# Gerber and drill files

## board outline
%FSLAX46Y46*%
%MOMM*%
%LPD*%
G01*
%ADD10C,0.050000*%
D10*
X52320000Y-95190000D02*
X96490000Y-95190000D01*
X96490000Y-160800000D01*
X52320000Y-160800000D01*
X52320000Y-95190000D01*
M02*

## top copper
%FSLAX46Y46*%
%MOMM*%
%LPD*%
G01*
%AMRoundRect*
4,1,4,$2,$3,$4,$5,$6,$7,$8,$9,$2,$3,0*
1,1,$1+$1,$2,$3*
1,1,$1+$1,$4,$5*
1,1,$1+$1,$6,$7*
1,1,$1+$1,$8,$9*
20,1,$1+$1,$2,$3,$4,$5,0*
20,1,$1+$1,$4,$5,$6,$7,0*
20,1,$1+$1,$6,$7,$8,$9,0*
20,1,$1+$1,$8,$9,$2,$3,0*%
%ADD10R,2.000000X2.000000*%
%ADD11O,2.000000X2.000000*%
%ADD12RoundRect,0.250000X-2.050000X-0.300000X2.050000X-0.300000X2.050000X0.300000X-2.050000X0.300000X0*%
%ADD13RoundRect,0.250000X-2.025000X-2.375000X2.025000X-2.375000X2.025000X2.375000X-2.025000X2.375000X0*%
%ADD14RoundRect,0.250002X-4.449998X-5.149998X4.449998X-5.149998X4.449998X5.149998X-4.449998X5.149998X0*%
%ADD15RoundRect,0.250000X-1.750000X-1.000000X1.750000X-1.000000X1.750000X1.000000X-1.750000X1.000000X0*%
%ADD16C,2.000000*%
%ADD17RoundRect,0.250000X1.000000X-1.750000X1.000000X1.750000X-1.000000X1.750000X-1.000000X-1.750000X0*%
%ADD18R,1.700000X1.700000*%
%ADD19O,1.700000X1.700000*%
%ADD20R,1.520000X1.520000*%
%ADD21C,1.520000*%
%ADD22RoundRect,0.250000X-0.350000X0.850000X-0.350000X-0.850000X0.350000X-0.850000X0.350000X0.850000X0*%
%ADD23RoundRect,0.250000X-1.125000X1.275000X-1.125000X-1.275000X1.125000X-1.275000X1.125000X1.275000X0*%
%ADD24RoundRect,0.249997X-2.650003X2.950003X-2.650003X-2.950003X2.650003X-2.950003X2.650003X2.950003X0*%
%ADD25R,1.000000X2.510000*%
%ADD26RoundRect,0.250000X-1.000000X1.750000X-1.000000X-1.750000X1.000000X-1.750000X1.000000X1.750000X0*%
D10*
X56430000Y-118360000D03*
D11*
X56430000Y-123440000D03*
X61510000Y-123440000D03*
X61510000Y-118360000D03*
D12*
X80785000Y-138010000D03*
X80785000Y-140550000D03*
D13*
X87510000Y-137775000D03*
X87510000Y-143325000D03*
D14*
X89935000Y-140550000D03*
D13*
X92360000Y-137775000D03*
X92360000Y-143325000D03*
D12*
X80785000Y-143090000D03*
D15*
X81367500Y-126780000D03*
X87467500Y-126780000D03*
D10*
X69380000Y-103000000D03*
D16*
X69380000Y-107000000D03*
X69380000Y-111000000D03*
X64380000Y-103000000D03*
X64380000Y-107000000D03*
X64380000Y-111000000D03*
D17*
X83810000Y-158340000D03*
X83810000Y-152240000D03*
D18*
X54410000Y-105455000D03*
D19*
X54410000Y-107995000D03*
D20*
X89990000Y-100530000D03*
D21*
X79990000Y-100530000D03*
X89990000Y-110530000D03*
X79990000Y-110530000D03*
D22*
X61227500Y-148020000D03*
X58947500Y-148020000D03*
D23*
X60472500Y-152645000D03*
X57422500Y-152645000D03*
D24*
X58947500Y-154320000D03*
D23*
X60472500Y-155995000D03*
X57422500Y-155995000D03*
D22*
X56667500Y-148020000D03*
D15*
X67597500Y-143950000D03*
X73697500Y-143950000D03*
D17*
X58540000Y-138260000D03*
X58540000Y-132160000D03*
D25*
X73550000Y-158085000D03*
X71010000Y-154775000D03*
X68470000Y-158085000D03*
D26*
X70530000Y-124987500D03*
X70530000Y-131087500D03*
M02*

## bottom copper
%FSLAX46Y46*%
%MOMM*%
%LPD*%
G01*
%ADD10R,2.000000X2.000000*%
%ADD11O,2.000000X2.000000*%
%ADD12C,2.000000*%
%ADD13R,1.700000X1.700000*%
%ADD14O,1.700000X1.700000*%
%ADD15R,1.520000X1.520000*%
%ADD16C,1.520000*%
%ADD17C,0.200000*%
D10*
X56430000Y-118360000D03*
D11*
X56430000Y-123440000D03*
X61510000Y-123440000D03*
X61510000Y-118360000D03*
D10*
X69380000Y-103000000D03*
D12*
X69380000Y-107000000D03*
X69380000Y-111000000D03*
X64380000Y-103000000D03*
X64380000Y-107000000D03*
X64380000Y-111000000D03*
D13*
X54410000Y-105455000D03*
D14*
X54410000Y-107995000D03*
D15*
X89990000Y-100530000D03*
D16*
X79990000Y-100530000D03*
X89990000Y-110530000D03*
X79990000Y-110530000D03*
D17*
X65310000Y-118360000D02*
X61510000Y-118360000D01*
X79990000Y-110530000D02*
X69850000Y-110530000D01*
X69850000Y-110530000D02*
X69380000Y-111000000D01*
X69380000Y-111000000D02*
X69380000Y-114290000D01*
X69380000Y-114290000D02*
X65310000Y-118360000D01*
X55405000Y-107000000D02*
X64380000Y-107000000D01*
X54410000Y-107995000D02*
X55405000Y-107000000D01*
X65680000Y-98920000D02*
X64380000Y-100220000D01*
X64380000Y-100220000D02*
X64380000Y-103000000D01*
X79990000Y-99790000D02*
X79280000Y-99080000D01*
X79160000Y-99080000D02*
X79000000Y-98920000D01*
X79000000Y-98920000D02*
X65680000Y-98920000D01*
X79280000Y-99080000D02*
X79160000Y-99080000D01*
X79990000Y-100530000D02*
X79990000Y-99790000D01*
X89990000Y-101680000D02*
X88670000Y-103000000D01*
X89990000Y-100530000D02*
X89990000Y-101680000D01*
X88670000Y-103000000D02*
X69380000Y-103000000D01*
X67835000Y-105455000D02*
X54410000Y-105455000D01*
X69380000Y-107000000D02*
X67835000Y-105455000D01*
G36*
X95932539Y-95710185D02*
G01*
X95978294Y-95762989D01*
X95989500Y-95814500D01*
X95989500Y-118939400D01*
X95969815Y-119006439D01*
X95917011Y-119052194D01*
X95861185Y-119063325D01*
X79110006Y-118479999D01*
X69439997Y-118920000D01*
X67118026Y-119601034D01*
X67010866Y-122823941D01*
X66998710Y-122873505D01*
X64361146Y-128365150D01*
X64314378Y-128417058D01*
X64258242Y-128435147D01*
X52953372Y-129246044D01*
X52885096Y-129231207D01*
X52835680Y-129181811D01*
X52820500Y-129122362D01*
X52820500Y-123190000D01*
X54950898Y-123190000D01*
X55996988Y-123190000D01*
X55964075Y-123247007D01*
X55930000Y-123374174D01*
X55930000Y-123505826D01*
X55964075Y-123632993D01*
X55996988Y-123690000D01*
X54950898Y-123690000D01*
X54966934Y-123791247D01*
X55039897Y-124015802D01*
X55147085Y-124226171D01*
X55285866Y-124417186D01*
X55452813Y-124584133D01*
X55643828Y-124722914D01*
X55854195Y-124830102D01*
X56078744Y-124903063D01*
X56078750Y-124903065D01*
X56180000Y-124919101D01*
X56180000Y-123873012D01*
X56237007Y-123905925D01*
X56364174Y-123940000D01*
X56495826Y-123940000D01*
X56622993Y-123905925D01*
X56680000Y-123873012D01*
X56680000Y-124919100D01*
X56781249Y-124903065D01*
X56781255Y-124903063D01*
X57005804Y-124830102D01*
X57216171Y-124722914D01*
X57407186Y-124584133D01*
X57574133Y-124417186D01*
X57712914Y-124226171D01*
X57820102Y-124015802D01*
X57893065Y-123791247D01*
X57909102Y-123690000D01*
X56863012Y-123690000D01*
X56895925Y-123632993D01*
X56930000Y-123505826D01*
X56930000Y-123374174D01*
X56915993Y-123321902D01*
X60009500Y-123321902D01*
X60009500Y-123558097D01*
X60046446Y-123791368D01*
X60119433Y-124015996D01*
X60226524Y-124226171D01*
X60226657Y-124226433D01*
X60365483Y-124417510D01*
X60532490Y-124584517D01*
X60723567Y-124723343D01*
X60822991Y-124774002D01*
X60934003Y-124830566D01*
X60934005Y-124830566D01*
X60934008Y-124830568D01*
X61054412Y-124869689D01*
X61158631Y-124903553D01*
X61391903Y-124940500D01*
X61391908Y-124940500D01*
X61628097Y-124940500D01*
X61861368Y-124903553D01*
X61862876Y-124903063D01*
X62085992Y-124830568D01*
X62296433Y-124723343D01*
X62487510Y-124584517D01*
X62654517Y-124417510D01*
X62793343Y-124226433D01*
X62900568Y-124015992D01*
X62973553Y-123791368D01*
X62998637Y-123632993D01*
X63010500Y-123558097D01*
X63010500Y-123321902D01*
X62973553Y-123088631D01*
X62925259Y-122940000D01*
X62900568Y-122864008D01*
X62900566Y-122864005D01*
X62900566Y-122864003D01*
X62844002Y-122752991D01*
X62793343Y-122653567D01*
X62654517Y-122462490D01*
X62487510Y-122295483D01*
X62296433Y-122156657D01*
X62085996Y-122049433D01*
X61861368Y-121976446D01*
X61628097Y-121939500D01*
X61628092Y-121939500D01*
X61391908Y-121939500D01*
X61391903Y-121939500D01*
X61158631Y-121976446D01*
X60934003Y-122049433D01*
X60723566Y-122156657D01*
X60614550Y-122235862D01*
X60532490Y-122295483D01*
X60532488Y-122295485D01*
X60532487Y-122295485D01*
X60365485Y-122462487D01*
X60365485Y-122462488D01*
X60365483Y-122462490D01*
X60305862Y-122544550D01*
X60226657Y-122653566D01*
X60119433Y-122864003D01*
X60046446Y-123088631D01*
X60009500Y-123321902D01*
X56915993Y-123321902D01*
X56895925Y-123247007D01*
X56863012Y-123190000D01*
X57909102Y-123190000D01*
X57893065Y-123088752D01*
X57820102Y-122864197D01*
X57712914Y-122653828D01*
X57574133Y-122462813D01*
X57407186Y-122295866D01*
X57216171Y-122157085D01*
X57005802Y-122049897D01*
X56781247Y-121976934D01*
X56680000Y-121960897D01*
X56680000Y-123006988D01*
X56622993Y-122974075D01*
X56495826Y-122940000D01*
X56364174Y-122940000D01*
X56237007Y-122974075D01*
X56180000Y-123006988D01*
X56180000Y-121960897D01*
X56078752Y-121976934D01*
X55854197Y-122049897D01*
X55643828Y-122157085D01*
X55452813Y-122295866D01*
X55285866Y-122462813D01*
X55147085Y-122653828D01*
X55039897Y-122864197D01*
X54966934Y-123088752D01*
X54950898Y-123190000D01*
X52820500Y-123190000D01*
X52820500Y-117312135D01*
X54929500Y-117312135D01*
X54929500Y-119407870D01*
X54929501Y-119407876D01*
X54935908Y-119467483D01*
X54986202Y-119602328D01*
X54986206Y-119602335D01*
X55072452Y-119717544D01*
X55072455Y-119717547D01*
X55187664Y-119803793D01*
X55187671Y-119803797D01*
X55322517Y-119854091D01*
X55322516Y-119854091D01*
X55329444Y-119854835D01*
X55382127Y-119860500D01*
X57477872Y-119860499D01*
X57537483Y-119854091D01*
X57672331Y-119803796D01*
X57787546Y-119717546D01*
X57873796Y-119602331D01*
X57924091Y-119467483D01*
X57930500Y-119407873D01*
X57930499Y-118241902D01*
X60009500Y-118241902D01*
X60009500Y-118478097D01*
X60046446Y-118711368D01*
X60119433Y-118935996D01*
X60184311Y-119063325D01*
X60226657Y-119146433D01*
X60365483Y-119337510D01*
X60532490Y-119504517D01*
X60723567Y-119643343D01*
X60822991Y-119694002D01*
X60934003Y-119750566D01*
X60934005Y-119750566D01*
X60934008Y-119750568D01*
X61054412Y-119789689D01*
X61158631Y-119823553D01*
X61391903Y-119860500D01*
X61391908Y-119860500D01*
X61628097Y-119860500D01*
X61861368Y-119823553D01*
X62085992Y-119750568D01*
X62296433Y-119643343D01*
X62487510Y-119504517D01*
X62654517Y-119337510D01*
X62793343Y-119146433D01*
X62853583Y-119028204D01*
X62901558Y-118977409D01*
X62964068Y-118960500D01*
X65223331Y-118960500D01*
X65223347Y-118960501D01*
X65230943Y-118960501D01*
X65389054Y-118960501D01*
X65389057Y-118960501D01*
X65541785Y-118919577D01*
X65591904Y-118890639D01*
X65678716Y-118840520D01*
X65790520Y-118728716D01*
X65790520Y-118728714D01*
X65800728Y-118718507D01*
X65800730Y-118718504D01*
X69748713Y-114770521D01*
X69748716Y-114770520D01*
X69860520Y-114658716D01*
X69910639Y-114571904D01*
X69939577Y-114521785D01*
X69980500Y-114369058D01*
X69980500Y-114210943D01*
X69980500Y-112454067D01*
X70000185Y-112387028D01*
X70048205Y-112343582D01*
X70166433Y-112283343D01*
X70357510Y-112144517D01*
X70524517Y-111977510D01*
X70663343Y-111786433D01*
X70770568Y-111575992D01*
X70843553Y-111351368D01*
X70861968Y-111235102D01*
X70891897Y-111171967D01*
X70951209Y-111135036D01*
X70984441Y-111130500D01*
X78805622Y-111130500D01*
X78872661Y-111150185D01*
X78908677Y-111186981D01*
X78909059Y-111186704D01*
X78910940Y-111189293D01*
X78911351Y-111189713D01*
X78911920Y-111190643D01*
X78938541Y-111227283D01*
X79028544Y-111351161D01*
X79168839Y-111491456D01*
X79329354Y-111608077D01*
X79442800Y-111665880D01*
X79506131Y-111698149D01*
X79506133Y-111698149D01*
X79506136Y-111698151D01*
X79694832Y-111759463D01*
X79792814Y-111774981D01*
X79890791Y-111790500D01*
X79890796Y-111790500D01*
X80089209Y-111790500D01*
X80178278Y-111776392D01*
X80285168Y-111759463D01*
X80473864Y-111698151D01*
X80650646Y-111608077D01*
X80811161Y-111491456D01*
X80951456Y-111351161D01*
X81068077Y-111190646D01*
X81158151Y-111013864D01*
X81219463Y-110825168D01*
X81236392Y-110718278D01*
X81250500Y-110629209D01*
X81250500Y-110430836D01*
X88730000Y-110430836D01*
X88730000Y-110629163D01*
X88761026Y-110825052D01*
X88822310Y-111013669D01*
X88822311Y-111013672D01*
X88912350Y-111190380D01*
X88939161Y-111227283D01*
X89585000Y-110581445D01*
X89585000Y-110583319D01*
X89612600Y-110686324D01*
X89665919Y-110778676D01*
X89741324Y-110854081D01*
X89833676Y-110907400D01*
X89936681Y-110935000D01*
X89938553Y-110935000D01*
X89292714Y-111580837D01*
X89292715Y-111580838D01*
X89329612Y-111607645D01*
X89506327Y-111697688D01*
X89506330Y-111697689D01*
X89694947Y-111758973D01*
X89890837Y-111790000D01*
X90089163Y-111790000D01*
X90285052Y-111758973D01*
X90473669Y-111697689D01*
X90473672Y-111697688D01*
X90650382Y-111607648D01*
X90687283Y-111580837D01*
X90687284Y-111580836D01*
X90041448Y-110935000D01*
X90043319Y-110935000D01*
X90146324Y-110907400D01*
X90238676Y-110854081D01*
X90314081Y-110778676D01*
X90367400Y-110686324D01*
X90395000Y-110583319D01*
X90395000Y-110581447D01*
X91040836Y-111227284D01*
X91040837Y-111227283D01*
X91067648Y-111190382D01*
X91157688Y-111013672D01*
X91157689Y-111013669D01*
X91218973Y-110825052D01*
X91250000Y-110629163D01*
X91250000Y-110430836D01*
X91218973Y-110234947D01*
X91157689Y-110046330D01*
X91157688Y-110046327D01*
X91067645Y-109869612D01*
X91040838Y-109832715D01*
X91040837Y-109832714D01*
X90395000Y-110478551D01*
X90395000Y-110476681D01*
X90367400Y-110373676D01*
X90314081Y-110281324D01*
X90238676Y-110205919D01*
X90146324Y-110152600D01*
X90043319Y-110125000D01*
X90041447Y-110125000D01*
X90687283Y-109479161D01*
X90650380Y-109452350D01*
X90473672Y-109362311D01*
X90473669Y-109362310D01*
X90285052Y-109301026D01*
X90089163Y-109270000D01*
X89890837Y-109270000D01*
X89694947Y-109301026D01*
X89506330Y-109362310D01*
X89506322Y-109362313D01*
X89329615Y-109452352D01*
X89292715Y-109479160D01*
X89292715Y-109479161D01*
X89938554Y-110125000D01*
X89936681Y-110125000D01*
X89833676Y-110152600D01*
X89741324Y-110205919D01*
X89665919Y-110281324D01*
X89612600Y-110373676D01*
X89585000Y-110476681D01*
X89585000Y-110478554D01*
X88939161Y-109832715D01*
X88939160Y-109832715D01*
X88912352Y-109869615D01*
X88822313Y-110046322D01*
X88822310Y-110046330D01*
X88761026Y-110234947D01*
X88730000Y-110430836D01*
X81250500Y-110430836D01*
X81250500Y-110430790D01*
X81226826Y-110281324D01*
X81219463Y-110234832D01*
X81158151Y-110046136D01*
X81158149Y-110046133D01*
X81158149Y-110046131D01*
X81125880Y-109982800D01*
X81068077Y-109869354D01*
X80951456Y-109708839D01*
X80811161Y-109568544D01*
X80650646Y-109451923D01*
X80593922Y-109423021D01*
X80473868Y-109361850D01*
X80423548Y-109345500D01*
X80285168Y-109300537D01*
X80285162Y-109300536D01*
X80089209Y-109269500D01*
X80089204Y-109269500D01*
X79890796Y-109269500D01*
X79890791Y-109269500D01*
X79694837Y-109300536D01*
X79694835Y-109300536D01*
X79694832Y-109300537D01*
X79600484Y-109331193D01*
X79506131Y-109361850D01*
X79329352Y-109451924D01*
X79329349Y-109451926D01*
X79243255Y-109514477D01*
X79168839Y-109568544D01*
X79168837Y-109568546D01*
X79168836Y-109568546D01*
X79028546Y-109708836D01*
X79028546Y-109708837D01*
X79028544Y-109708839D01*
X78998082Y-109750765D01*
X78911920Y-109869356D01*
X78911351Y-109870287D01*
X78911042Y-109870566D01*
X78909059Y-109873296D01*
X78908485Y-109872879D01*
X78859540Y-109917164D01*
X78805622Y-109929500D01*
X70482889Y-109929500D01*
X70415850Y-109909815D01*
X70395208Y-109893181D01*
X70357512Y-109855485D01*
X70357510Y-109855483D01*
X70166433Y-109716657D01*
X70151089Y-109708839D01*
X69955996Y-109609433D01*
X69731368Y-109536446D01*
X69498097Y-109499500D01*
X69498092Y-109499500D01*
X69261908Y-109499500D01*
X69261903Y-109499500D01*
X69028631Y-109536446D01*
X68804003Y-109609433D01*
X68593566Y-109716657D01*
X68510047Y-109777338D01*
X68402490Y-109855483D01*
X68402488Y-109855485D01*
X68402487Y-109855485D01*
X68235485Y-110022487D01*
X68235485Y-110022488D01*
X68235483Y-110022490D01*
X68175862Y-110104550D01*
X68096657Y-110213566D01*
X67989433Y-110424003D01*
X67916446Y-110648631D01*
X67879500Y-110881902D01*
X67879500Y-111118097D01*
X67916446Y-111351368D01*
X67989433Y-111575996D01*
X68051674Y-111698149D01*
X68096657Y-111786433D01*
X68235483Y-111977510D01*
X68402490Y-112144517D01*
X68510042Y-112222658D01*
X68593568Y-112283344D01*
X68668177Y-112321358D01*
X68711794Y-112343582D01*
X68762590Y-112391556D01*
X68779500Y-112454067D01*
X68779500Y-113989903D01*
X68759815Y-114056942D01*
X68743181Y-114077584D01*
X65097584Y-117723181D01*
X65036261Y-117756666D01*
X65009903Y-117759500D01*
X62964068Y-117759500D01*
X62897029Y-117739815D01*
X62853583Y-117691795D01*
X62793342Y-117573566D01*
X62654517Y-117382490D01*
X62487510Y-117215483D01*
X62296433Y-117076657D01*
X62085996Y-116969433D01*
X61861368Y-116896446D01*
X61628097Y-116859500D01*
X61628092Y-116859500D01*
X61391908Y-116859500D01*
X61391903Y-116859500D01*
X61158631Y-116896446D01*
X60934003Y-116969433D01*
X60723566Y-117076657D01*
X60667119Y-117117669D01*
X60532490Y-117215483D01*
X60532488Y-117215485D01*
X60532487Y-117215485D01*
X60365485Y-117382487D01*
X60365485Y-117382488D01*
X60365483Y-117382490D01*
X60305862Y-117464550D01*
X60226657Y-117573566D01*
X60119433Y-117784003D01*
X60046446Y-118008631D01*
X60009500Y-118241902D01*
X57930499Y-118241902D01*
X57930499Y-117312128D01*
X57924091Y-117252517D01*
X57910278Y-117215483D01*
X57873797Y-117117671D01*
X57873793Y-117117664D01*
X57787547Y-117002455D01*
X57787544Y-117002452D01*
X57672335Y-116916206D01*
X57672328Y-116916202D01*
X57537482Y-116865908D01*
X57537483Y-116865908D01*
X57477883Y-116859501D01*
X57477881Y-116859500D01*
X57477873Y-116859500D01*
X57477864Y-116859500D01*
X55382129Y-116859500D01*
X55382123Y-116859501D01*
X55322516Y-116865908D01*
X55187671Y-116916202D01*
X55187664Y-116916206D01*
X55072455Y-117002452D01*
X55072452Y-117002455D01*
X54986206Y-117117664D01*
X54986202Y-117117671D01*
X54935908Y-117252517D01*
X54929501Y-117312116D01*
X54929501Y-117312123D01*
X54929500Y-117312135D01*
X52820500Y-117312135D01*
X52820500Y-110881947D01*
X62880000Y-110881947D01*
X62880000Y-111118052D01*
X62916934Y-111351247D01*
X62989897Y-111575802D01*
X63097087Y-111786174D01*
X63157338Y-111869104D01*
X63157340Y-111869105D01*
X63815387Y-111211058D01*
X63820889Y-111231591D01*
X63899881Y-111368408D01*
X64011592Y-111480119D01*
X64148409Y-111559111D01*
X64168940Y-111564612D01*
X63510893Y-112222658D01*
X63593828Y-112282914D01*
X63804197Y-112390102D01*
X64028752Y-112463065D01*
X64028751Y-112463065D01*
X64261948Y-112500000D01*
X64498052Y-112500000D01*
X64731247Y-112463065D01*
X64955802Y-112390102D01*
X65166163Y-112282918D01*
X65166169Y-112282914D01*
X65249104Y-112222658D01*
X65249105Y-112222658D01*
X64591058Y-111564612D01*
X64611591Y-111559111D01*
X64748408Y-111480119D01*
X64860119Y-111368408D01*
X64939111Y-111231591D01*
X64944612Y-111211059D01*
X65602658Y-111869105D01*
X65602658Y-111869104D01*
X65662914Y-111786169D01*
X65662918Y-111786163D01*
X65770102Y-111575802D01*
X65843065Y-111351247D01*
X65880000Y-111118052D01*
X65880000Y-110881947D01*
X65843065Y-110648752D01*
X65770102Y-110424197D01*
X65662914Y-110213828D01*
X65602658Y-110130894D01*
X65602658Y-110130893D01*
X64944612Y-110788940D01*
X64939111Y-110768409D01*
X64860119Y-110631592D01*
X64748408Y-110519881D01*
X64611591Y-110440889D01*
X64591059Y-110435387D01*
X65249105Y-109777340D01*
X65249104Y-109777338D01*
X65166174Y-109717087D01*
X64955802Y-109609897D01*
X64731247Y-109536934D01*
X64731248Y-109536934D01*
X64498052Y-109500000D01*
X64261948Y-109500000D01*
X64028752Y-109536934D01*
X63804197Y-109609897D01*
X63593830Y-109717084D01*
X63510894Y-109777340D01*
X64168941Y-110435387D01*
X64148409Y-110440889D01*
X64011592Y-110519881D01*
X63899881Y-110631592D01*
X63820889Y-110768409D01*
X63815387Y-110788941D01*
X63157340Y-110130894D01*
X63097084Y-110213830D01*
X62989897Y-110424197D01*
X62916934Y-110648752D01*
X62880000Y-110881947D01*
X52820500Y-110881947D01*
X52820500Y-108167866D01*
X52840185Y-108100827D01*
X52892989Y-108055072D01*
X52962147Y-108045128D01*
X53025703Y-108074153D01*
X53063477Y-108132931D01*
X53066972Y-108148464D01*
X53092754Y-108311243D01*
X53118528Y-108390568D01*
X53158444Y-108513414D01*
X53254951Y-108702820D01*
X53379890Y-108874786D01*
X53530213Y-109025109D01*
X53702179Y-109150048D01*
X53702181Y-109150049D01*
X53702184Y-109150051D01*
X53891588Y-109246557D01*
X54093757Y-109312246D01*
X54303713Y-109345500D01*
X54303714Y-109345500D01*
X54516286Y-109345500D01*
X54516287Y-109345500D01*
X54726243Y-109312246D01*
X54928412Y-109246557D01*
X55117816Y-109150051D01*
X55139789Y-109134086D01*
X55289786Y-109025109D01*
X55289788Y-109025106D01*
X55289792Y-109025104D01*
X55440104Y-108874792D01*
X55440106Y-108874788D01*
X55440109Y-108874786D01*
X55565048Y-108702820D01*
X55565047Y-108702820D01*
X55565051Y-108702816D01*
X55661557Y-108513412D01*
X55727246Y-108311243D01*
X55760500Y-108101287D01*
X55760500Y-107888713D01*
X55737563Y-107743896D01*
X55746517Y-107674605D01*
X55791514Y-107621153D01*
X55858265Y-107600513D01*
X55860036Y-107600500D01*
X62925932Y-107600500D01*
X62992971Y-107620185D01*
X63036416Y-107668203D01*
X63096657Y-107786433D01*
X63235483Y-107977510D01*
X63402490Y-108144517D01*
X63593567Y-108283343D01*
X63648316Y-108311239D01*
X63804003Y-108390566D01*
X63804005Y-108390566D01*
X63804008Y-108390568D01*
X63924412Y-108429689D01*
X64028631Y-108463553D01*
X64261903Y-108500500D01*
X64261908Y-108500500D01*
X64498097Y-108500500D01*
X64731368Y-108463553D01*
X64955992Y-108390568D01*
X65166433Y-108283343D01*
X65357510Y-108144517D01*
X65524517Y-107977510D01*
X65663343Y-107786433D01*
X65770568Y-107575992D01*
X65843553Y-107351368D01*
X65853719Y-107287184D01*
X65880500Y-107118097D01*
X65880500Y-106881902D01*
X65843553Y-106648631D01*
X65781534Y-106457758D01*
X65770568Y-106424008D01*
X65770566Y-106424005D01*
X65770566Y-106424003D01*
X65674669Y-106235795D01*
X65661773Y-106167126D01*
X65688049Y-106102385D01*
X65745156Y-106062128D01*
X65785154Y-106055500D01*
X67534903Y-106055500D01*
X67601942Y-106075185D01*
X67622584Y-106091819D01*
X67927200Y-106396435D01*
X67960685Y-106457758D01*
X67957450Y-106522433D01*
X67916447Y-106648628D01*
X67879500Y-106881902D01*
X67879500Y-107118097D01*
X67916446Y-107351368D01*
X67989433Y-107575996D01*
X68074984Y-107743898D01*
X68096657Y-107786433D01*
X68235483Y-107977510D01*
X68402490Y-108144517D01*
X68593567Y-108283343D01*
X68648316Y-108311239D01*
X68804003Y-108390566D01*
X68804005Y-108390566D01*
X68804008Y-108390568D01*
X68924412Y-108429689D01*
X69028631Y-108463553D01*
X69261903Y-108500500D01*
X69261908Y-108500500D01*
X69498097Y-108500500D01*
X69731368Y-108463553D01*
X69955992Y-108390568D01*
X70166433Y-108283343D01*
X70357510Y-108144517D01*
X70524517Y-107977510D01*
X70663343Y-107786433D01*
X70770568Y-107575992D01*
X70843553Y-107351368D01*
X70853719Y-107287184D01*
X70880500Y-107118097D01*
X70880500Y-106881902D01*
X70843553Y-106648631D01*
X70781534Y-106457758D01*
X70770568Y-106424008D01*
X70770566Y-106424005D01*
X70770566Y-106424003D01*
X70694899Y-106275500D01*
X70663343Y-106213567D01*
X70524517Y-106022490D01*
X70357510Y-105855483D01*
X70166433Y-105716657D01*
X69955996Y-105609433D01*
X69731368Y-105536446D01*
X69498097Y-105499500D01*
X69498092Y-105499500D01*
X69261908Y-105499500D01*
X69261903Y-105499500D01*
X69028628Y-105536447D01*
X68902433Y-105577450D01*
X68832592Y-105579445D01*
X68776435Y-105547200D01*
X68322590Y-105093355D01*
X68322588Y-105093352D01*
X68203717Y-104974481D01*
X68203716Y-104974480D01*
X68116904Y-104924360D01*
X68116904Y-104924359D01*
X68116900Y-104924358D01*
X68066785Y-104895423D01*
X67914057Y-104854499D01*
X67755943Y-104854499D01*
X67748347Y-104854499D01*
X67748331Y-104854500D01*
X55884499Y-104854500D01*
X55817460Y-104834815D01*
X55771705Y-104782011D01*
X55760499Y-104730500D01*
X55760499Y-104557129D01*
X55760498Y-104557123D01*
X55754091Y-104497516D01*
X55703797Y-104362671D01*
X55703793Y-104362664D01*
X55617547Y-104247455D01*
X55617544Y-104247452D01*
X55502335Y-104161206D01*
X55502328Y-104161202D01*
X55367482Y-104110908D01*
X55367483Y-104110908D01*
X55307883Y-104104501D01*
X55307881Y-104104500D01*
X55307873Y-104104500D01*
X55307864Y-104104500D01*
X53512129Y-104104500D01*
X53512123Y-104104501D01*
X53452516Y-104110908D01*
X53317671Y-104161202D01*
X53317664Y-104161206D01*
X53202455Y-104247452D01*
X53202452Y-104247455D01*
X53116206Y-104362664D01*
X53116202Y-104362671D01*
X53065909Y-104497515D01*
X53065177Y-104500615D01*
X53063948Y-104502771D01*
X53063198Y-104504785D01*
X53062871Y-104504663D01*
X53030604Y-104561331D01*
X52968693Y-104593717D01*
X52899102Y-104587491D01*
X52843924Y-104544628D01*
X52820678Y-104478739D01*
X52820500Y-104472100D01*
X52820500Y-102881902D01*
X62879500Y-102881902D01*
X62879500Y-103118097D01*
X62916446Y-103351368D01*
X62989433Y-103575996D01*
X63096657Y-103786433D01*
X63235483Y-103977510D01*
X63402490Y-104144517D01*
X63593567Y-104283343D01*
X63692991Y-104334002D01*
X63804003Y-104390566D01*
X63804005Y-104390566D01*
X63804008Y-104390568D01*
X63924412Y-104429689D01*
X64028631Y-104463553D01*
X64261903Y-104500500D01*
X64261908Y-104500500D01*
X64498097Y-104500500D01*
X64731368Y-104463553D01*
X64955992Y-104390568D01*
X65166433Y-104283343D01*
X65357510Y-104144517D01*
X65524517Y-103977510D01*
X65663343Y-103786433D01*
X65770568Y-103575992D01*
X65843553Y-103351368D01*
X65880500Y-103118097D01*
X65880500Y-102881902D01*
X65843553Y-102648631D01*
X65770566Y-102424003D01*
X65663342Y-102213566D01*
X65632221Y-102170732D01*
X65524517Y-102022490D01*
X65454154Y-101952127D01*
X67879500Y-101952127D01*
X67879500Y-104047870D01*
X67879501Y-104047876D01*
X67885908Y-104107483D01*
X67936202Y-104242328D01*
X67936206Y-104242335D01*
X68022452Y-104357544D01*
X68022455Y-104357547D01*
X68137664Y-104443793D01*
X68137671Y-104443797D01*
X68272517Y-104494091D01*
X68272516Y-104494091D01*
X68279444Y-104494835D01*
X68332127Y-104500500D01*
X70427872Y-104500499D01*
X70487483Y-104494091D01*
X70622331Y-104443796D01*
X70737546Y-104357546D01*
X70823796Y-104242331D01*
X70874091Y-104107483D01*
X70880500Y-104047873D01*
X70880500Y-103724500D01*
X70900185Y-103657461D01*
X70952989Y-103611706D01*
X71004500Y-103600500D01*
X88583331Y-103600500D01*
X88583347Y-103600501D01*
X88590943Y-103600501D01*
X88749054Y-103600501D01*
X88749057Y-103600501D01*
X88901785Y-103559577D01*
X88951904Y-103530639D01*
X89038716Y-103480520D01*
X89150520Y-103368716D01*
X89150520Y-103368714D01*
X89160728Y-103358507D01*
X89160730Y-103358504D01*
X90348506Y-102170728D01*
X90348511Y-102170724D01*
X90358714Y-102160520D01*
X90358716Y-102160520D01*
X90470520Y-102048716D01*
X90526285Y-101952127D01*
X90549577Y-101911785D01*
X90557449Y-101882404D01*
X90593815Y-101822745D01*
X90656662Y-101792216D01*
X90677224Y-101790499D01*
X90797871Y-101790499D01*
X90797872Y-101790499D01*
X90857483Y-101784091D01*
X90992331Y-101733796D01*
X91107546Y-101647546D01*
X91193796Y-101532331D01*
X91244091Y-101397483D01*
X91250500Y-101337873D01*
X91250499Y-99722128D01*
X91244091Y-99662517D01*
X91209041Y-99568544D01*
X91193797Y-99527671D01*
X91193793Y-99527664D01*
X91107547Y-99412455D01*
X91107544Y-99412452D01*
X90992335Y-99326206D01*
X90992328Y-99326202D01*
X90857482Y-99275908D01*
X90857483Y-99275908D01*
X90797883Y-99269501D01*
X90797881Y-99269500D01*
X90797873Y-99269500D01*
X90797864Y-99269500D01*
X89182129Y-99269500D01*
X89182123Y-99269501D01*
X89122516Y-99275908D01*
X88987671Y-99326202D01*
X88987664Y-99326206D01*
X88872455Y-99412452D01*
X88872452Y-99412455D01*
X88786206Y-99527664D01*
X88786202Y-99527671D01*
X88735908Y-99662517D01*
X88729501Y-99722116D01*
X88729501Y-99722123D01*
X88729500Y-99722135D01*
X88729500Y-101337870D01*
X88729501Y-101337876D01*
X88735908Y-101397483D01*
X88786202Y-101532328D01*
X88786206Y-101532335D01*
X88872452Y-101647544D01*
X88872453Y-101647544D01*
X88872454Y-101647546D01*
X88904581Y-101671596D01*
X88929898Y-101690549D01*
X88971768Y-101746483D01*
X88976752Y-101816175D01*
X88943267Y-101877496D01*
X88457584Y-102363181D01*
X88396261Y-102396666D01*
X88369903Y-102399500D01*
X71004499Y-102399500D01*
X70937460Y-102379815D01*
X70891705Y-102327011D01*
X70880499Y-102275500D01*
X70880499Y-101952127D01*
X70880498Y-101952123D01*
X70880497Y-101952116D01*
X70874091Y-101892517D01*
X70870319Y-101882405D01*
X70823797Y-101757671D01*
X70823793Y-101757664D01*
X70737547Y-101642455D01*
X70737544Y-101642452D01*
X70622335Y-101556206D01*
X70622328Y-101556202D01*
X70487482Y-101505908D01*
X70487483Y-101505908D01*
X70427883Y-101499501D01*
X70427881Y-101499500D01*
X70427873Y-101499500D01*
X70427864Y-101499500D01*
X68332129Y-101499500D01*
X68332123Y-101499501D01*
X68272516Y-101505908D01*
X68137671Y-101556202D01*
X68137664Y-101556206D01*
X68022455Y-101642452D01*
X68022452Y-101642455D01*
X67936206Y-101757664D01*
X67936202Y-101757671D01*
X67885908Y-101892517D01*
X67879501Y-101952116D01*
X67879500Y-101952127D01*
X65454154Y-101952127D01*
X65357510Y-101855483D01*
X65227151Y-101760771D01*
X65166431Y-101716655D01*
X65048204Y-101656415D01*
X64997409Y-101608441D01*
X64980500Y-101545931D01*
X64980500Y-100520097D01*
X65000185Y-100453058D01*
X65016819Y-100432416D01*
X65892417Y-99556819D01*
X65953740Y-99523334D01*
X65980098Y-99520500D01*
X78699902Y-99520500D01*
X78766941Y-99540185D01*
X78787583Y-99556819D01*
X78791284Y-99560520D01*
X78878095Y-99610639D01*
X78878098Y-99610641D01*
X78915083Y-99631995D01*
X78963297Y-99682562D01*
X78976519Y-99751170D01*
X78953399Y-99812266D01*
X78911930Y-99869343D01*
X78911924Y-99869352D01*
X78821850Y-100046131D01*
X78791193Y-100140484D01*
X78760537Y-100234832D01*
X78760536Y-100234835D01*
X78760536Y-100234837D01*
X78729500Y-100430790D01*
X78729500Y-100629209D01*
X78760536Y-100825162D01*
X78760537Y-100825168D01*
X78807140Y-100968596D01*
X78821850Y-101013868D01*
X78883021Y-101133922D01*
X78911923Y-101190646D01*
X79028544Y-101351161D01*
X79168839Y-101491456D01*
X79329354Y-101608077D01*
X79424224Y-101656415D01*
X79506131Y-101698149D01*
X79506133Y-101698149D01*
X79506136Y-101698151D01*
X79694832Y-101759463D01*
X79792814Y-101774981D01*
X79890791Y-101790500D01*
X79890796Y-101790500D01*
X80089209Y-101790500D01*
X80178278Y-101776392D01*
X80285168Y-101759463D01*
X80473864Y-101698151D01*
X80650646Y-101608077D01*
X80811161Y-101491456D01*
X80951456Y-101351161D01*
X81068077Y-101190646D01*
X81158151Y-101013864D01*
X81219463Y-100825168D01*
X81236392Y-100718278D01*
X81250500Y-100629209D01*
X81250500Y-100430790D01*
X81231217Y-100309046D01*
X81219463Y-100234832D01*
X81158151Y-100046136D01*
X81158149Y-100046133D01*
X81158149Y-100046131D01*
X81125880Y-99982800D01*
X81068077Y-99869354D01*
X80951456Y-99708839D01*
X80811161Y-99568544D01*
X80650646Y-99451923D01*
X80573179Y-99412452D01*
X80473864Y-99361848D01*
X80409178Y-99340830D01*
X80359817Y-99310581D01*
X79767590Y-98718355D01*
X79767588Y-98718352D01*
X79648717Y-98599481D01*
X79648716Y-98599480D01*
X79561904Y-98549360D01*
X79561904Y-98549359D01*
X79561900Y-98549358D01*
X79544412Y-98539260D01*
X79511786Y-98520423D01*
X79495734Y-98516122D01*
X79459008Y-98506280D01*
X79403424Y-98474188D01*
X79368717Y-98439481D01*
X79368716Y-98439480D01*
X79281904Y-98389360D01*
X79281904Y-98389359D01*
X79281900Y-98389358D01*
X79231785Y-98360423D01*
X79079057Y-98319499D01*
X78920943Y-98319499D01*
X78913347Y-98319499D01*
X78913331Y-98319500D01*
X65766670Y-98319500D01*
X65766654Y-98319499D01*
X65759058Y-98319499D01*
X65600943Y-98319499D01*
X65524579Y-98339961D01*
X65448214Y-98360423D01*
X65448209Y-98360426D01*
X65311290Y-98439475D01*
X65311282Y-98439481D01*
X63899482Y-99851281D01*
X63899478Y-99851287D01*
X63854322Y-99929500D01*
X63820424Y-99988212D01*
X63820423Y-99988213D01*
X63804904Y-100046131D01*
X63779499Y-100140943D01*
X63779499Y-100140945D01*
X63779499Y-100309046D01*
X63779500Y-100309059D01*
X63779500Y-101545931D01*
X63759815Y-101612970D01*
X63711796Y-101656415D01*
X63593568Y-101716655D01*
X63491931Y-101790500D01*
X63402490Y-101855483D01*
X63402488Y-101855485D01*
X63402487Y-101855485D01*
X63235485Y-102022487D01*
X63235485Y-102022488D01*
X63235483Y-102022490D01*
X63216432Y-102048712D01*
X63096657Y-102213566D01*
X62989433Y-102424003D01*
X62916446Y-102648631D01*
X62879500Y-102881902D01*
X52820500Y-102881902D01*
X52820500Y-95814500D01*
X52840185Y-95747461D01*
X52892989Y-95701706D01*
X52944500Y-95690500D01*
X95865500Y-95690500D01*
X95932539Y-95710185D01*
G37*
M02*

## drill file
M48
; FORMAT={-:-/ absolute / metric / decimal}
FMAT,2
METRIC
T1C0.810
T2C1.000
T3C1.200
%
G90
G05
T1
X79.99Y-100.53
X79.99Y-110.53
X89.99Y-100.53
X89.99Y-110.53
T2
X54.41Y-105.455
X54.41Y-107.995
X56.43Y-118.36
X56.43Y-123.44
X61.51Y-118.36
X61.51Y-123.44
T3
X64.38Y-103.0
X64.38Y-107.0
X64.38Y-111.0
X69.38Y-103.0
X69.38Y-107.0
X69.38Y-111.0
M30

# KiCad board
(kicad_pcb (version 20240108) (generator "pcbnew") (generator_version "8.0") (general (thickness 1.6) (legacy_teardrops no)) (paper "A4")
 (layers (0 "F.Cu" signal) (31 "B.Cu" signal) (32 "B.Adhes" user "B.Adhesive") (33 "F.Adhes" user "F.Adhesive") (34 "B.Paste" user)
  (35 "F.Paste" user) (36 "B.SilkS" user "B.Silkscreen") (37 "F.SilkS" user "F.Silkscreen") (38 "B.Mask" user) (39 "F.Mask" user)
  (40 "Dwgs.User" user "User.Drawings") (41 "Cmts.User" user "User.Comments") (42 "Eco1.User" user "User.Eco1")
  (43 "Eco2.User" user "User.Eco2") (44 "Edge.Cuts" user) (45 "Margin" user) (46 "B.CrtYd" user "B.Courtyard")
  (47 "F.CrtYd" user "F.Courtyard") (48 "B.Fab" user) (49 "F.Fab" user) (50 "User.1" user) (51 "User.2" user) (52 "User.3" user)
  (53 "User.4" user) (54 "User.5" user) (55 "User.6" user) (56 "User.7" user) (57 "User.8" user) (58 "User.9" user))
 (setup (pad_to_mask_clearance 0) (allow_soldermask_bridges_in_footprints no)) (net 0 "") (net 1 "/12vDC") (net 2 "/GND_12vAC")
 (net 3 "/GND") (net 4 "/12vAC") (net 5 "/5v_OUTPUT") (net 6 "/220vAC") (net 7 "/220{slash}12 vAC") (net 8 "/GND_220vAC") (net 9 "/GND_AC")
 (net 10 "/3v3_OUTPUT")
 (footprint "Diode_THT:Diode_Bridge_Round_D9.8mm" (layer "F.Cu") (at 56.43 118.36)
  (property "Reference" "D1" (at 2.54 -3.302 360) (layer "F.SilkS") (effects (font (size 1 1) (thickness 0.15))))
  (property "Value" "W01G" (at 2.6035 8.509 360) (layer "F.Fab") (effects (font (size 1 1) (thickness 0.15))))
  (pad "1" thru_hole rect (at 0 0) (size 2 2) (drill 1) (layers "*.Cu" "*.Mask") (remove_unused_layers no) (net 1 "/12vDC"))
  (pad "2" thru_hole oval (at 0 5.08) (size 2 2) (drill 1) (layers "*.Cu" "*.Mask") (remove_unused_layers no) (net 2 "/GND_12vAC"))
  (pad "3" thru_hole oval (at 5.08 5.08) (size 2 2) (drill 1) (layers "*.Cu" "*.Mask") (remove_unused_layers no) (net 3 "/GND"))
  (pad "4" thru_hole oval (at 5.08 0) (size 2 2) (drill 1) (layers "*.Cu" "*.Mask") (remove_unused_layers no) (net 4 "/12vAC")))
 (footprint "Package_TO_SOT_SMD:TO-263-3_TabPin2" (layer "F.Cu") (at 88.435 140.55)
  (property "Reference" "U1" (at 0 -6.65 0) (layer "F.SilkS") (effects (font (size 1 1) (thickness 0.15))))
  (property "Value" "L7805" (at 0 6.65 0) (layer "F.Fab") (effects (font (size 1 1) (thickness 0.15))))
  (pad "1" smd roundrect (at -7.65 -2.54) (size 4.6 1.1) (layers "F.Cu" "F.Paste" "F.Mask") (roundrect_rratio 0.227273) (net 1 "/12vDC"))
  (pad "2" smd roundrect (at -7.65 0) (size 4.6 1.1) (layers "F.Cu" "F.Paste" "F.Mask") (roundrect_rratio 0.227273) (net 3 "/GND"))
  (pad "2" smd roundrect (at -0.925 -2.775) (size 4.55 5.25) (layers "F.Cu" "F.Paste") (roundrect_rratio 0.054945) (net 3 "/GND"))
  (pad "2" smd roundrect (at -0.925 2.775) (size 4.55 5.25) (layers "F.Cu" "F.Paste") (roundrect_rratio 0.054945) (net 3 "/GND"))
  (pad "2" smd roundrect (at 1.5 0) (size 9.4 10.8) (layers "F.Cu" "F.Mask") (roundrect_rratio 0.026596) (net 3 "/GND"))
  (pad "2" smd roundrect (at 3.925 -2.775) (size 4.55 5.25) (layers "F.Cu" "F.Paste") (roundrect_rratio 0.054945) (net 3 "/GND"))
  (pad "2" smd roundrect (at 3.925 2.775) (size 4.55 5.25) (layers "F.Cu" "F.Paste") (roundrect_rratio 0.054945) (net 3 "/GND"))
  (pad "3" smd roundrect (at -7.65 2.54) (size 4.6 1.1) (layers "F.Cu" "F.Paste" "F.Mask") (roundrect_rratio 0.227273) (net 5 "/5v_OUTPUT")))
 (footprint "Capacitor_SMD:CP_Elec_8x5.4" (layer "F.Cu") (at 84.4175 126.78)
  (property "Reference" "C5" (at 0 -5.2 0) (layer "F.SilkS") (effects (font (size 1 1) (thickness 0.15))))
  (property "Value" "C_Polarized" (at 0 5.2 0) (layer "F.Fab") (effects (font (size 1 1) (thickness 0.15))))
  (pad "1" smd roundrect (at -3.05 0) (size 4 2.5) (layers "F.Cu" "F.Paste" "F.Mask") (roundrect_rratio 0.1) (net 5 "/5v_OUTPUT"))
  (pad "2" smd roundrect (at 3.05 0) (size 4 2.5) (layers "F.Cu" "F.Paste" "F.Mask") (roundrect_rratio 0.1) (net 3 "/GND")))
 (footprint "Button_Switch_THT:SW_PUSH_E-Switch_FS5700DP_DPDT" (layer "F.Cu") (at 69.38 103 -90)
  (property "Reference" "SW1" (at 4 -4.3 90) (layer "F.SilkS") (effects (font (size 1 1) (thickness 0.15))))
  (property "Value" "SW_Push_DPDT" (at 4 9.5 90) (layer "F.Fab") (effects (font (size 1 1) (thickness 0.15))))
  (pad "1" thru_hole rect (at 0 0 270) (size 2 2) (drill 1.2) (layers "*.Cu" "*.Mask") (remove_unused_layers no) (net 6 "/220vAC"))
  (pad "2" thru_hole circle (at 4 0 270) (size 2 2) (drill 1.2) (layers "*.Cu" "*.Mask") (remove_unused_layers no)
   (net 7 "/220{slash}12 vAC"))
  (pad "3" thru_hole circle (at 8 0 270) (size 2 2) (drill 1.2) (layers "*.Cu" "*.Mask") (remove_unused_layers no) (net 4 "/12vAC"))
  (pad "4" thru_hole circle (at 0 5 270) (size 2 2) (drill 1.2) (layers "*.Cu" "*.Mask") (remove_unused_layers no) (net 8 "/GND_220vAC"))
  (pad "5" thru_hole circle (at 4 5 270) (size 2 2) (drill 1.2) (layers "*.Cu" "*.Mask") (remove_unused_layers no) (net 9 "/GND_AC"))
  (pad "6" thru_hole circle (at 8 5 270) (size 2 2) (drill 1.2) (layers "*.Cu" "*.Mask") (remove_unused_layers no) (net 2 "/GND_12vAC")))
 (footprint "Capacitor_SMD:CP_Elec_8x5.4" (layer "F.Cu") (at 83.81 155.29 90)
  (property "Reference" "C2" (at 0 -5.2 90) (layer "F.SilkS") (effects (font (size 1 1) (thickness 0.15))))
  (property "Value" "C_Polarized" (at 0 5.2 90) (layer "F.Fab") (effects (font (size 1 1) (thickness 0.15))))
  (pad "1" smd roundrect (at -3.05 0 90) (size 4 2.5) (layers "F.Cu" "F.Paste" "F.Mask") (roundrect_rratio 0.1) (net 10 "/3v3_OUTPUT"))
  (pad "2" smd roundrect (at 3.05 0 90) (size 4 2.5) (layers "F.Cu" "F.Paste" "F.Mask") (roundrect_rratio 0.1) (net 3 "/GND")))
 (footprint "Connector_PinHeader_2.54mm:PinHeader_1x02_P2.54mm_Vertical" (layer "F.Cu") (at 54.41 105.455)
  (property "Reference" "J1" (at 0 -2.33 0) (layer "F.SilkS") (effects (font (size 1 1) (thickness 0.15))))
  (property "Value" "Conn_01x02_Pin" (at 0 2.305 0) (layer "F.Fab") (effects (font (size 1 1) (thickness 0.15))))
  (pad "1" thru_hole rect (at 0 0) (size 1.7 1.7) (drill 1) (layers "*.Cu" "*.Mask") (remove_unused_layers no) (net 7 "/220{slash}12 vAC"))
  (pad "2" thru_hole oval (at 0 2.54) (size 1.7 1.7) (drill 1) (layers "*.Cu" "*.Mask") (remove_unused_layers no) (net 9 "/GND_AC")))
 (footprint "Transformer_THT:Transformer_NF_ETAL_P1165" (layer "F.Cu") (at 89.99 100.53)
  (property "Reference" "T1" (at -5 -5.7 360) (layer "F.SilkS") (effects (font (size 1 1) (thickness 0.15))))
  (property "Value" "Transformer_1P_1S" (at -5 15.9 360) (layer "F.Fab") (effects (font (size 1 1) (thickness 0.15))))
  (pad "1" thru_hole rect (at 0 0) (size 1.52 1.52) (drill 0.81) (layers "*.Cu" "*.Mask") (remove_unused_layers no) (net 6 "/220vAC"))
  (pad "2" thru_hole circle (at -10 0) (size 1.52 1.52) (drill 0.81) (layers "*.Cu" "*.Mask") (remove_unused_layers no)
   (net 8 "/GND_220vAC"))
  (pad "3" thru_hole circle (at 0 10) (size 1.52 1.52) (drill 0.81) (layers "*.Cu" "*.Mask") (remove_unused_layers no) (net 2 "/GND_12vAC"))
  (pad "4" thru_hole circle (at -10 10) (size 1.52 1.52) (drill 0.81) (layers "*.Cu" "*.Mask") (remove_unused_layers no) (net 4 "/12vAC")))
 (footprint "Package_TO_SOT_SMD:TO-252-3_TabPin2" (layer "F.Cu") (at 58.9475 153.06 -90)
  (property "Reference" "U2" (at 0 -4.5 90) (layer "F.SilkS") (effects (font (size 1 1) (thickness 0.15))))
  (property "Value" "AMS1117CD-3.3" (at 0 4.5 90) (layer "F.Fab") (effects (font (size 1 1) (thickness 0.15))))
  (pad "1" smd roundrect (at -5.04 -2.28 270) (size 2.2 1.2) (layers "F.Cu" "F.Paste" "F.Mask") (roundrect_rratio 0.208333) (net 3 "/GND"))
  (pad "2" smd roundrect (at -5.04 0 270) (size 2.2 1.2) (layers "F.Cu" "F.Paste" "F.Mask") (roundrect_rratio 0.208333)
   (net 10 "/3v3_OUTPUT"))
  (pad "2" smd roundrect (at -0.415 -1.525 270) (size 3.05 2.75) (layers "F.Cu" "F.Paste") (roundrect_rratio 0.090909)
   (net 10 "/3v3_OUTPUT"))
  (pad "2" smd roundrect (at -0.415 1.525 270) (size 3.05 2.75) (layers "F.Cu" "F.Paste") (roundrect_rratio 0.090909) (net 10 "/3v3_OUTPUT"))
  (pad "2" smd roundrect (at 1.26 0 270) (size 6.4 5.8) (layers "F.Cu" "F.Mask") (roundrect_rratio 0.043103) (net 10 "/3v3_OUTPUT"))
  (pad "2" smd roundrect (at 2.935 -1.525 270) (size 3.05 2.75) (layers "F.Cu" "F.Paste") (roundrect_rratio 0.090909) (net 10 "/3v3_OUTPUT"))
  (pad "2" smd roundrect (at 2.935 1.525 270) (size 3.05 2.75) (layers "F.Cu" "F.Paste") (roundrect_rratio 0.090909) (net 10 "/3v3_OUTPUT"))
  (pad "3" smd roundrect (at -5.04 2.28 270) (size 2.2 1.2) (layers "F.Cu" "F.Paste" "F.Mask") (roundrect_rratio 0.208333)
   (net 5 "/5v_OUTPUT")))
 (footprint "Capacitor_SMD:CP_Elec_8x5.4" (layer "F.Cu") (at 70.6475 143.95)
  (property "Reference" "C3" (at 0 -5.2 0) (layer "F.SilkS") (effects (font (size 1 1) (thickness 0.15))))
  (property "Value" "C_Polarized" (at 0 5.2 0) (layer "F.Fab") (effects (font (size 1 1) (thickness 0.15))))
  (pad "1" smd roundrect (at -3.05 0) (size 4 2.5) (layers "F.Cu" "F.Paste" "F.Mask") (roundrect_rratio 0.1) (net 10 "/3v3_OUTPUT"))
  (pad "2" smd roundrect (at 3.05 0) (size 4 2.5) (layers "F.Cu" "F.Paste" "F.Mask") (roundrect_rratio 0.1) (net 3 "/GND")))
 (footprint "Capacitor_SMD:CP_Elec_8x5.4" (layer "F.Cu") (at 58.54 135.21 90)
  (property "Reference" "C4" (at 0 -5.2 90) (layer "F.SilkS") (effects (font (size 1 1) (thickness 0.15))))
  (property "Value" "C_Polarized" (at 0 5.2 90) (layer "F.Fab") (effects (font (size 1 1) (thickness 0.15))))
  (pad "1" smd roundrect (at -3.05 0 90) (size 4 2.5) (layers "F.Cu" "F.Paste" "F.Mask") (roundrect_rratio 0.1) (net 5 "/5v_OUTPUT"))
  (pad "2" smd roundrect (at 3.05 0 90) (size 4 2.5) (layers "F.Cu" "F.Paste" "F.Mask") (roundrect_rratio 0.1) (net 3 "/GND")))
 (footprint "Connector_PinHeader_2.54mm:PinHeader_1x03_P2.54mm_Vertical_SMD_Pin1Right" (layer "F.Cu") (at 71.01 156.43 -90)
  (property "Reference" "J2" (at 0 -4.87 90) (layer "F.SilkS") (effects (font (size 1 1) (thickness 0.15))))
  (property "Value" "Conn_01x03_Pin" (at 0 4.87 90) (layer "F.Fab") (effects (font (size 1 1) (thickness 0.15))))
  (pad "1" smd rect (at 1.655 -2.54 270) (size 2.51 1) (layers "F.Cu" "F.Paste" "F.Mask") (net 3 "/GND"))
  (pad "2" smd rect (at -1.655 0 270) (size 2.51 1) (layers "F.Cu" "F.Paste" "F.Mask") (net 5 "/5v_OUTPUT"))
  (pad "3" smd rect (at 1.655 2.54 270) (size 2.51 1) (layers "F.Cu" "F.Paste" "F.Mask") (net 10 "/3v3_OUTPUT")))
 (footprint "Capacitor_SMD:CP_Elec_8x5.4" (layer "F.Cu") (at 70.53 128.0375 -90)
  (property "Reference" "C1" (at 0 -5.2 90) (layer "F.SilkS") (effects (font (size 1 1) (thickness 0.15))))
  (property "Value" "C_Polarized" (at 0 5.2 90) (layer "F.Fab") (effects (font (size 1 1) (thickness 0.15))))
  (pad "1" smd roundrect (at -3.05 0 270) (size 4 2.5) (layers "F.Cu" "F.Paste" "F.Mask") (roundrect_rratio 0.1) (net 1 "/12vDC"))
  (pad "2" smd roundrect (at 3.05 0 270) (size 4 2.5) (layers "F.Cu" "F.Paste" "F.Mask") (roundrect_rratio 0.1) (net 3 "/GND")))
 (gr_rect (start 52.32 95.19) (end 96.49 160.8) (stroke (width 0.05) (type default)) (fill none) (layer "Edge.Cuts"))
 (segment (start 65.31 118.36) (end 61.51 118.36) (width 0.2) (layer "B.Cu") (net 4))
 (segment (start 79.99 110.53) (end 69.85 110.53) (width 0.2) (layer "B.Cu") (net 4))
 (segment (start 69.85 110.53) (end 69.38 111) (width 0.2) (layer "B.Cu") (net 4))
 (segment (start 69.38 111) (end 69.38 114.29) (width 0.2) (layer "B.Cu") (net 4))
 (segment (start 69.38 114.29) (end 65.31 118.36) (width 0.2) (layer "B.Cu") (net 4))
 (segment (start 55.405 107) (end 64.38 107) (width 0.2) (layer "B.Cu") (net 9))
 (segment (start 54.41 107.995) (end 55.405 107) (width 0.2) (layer "B.Cu") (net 9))
 (segment (start 65.68 98.92) (end 64.38 100.22) (width 0.2) (layer "B.Cu") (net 8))
 (segment (start 64.38 100.22) (end 64.38 103) (width 0.2) (layer "B.Cu") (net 8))
 (segment (start 79.99 99.79) (end 79.28 99.08) (width 0.2) (layer "B.Cu") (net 8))
 (segment (start 79.16 99.08) (end 79 98.92) (width 0.2) (layer "B.Cu") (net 8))
 (segment (start 79 98.92) (end 65.68 98.92) (width 0.2) (layer "B.Cu") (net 8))
 (segment (start 79.28 99.08) (end 79.16 99.08) (width 0.2) (layer "B.Cu") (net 8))
 (segment (start 79.99 100.53) (end 79.99 99.79) (width 0.2) (layer "B.Cu") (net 8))
 (segment (start 89.99 101.68) (end 88.67 103) (width 0.2) (layer "B.Cu") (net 6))
 (segment (start 89.99 100.53) (end 89.99 101.68) (width 0.2) (layer "B.Cu") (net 6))
 (segment (start 88.67 103) (end 69.38 103) (width 0.2) (layer "B.Cu") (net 6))
 (segment (start 67.835 105.455) (end 54.41 105.455) (width 0.2) (layer "B.Cu") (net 7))
 (segment (start 69.38 107) (end 67.835 105.455) (width 0.2) (layer "B.Cu") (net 7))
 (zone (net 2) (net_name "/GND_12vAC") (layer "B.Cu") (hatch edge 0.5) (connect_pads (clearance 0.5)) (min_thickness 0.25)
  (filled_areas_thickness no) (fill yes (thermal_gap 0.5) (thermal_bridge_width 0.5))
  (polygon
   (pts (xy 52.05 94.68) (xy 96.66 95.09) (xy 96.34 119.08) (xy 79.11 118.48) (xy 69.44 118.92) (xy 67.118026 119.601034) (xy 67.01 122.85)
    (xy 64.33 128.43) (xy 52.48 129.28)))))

